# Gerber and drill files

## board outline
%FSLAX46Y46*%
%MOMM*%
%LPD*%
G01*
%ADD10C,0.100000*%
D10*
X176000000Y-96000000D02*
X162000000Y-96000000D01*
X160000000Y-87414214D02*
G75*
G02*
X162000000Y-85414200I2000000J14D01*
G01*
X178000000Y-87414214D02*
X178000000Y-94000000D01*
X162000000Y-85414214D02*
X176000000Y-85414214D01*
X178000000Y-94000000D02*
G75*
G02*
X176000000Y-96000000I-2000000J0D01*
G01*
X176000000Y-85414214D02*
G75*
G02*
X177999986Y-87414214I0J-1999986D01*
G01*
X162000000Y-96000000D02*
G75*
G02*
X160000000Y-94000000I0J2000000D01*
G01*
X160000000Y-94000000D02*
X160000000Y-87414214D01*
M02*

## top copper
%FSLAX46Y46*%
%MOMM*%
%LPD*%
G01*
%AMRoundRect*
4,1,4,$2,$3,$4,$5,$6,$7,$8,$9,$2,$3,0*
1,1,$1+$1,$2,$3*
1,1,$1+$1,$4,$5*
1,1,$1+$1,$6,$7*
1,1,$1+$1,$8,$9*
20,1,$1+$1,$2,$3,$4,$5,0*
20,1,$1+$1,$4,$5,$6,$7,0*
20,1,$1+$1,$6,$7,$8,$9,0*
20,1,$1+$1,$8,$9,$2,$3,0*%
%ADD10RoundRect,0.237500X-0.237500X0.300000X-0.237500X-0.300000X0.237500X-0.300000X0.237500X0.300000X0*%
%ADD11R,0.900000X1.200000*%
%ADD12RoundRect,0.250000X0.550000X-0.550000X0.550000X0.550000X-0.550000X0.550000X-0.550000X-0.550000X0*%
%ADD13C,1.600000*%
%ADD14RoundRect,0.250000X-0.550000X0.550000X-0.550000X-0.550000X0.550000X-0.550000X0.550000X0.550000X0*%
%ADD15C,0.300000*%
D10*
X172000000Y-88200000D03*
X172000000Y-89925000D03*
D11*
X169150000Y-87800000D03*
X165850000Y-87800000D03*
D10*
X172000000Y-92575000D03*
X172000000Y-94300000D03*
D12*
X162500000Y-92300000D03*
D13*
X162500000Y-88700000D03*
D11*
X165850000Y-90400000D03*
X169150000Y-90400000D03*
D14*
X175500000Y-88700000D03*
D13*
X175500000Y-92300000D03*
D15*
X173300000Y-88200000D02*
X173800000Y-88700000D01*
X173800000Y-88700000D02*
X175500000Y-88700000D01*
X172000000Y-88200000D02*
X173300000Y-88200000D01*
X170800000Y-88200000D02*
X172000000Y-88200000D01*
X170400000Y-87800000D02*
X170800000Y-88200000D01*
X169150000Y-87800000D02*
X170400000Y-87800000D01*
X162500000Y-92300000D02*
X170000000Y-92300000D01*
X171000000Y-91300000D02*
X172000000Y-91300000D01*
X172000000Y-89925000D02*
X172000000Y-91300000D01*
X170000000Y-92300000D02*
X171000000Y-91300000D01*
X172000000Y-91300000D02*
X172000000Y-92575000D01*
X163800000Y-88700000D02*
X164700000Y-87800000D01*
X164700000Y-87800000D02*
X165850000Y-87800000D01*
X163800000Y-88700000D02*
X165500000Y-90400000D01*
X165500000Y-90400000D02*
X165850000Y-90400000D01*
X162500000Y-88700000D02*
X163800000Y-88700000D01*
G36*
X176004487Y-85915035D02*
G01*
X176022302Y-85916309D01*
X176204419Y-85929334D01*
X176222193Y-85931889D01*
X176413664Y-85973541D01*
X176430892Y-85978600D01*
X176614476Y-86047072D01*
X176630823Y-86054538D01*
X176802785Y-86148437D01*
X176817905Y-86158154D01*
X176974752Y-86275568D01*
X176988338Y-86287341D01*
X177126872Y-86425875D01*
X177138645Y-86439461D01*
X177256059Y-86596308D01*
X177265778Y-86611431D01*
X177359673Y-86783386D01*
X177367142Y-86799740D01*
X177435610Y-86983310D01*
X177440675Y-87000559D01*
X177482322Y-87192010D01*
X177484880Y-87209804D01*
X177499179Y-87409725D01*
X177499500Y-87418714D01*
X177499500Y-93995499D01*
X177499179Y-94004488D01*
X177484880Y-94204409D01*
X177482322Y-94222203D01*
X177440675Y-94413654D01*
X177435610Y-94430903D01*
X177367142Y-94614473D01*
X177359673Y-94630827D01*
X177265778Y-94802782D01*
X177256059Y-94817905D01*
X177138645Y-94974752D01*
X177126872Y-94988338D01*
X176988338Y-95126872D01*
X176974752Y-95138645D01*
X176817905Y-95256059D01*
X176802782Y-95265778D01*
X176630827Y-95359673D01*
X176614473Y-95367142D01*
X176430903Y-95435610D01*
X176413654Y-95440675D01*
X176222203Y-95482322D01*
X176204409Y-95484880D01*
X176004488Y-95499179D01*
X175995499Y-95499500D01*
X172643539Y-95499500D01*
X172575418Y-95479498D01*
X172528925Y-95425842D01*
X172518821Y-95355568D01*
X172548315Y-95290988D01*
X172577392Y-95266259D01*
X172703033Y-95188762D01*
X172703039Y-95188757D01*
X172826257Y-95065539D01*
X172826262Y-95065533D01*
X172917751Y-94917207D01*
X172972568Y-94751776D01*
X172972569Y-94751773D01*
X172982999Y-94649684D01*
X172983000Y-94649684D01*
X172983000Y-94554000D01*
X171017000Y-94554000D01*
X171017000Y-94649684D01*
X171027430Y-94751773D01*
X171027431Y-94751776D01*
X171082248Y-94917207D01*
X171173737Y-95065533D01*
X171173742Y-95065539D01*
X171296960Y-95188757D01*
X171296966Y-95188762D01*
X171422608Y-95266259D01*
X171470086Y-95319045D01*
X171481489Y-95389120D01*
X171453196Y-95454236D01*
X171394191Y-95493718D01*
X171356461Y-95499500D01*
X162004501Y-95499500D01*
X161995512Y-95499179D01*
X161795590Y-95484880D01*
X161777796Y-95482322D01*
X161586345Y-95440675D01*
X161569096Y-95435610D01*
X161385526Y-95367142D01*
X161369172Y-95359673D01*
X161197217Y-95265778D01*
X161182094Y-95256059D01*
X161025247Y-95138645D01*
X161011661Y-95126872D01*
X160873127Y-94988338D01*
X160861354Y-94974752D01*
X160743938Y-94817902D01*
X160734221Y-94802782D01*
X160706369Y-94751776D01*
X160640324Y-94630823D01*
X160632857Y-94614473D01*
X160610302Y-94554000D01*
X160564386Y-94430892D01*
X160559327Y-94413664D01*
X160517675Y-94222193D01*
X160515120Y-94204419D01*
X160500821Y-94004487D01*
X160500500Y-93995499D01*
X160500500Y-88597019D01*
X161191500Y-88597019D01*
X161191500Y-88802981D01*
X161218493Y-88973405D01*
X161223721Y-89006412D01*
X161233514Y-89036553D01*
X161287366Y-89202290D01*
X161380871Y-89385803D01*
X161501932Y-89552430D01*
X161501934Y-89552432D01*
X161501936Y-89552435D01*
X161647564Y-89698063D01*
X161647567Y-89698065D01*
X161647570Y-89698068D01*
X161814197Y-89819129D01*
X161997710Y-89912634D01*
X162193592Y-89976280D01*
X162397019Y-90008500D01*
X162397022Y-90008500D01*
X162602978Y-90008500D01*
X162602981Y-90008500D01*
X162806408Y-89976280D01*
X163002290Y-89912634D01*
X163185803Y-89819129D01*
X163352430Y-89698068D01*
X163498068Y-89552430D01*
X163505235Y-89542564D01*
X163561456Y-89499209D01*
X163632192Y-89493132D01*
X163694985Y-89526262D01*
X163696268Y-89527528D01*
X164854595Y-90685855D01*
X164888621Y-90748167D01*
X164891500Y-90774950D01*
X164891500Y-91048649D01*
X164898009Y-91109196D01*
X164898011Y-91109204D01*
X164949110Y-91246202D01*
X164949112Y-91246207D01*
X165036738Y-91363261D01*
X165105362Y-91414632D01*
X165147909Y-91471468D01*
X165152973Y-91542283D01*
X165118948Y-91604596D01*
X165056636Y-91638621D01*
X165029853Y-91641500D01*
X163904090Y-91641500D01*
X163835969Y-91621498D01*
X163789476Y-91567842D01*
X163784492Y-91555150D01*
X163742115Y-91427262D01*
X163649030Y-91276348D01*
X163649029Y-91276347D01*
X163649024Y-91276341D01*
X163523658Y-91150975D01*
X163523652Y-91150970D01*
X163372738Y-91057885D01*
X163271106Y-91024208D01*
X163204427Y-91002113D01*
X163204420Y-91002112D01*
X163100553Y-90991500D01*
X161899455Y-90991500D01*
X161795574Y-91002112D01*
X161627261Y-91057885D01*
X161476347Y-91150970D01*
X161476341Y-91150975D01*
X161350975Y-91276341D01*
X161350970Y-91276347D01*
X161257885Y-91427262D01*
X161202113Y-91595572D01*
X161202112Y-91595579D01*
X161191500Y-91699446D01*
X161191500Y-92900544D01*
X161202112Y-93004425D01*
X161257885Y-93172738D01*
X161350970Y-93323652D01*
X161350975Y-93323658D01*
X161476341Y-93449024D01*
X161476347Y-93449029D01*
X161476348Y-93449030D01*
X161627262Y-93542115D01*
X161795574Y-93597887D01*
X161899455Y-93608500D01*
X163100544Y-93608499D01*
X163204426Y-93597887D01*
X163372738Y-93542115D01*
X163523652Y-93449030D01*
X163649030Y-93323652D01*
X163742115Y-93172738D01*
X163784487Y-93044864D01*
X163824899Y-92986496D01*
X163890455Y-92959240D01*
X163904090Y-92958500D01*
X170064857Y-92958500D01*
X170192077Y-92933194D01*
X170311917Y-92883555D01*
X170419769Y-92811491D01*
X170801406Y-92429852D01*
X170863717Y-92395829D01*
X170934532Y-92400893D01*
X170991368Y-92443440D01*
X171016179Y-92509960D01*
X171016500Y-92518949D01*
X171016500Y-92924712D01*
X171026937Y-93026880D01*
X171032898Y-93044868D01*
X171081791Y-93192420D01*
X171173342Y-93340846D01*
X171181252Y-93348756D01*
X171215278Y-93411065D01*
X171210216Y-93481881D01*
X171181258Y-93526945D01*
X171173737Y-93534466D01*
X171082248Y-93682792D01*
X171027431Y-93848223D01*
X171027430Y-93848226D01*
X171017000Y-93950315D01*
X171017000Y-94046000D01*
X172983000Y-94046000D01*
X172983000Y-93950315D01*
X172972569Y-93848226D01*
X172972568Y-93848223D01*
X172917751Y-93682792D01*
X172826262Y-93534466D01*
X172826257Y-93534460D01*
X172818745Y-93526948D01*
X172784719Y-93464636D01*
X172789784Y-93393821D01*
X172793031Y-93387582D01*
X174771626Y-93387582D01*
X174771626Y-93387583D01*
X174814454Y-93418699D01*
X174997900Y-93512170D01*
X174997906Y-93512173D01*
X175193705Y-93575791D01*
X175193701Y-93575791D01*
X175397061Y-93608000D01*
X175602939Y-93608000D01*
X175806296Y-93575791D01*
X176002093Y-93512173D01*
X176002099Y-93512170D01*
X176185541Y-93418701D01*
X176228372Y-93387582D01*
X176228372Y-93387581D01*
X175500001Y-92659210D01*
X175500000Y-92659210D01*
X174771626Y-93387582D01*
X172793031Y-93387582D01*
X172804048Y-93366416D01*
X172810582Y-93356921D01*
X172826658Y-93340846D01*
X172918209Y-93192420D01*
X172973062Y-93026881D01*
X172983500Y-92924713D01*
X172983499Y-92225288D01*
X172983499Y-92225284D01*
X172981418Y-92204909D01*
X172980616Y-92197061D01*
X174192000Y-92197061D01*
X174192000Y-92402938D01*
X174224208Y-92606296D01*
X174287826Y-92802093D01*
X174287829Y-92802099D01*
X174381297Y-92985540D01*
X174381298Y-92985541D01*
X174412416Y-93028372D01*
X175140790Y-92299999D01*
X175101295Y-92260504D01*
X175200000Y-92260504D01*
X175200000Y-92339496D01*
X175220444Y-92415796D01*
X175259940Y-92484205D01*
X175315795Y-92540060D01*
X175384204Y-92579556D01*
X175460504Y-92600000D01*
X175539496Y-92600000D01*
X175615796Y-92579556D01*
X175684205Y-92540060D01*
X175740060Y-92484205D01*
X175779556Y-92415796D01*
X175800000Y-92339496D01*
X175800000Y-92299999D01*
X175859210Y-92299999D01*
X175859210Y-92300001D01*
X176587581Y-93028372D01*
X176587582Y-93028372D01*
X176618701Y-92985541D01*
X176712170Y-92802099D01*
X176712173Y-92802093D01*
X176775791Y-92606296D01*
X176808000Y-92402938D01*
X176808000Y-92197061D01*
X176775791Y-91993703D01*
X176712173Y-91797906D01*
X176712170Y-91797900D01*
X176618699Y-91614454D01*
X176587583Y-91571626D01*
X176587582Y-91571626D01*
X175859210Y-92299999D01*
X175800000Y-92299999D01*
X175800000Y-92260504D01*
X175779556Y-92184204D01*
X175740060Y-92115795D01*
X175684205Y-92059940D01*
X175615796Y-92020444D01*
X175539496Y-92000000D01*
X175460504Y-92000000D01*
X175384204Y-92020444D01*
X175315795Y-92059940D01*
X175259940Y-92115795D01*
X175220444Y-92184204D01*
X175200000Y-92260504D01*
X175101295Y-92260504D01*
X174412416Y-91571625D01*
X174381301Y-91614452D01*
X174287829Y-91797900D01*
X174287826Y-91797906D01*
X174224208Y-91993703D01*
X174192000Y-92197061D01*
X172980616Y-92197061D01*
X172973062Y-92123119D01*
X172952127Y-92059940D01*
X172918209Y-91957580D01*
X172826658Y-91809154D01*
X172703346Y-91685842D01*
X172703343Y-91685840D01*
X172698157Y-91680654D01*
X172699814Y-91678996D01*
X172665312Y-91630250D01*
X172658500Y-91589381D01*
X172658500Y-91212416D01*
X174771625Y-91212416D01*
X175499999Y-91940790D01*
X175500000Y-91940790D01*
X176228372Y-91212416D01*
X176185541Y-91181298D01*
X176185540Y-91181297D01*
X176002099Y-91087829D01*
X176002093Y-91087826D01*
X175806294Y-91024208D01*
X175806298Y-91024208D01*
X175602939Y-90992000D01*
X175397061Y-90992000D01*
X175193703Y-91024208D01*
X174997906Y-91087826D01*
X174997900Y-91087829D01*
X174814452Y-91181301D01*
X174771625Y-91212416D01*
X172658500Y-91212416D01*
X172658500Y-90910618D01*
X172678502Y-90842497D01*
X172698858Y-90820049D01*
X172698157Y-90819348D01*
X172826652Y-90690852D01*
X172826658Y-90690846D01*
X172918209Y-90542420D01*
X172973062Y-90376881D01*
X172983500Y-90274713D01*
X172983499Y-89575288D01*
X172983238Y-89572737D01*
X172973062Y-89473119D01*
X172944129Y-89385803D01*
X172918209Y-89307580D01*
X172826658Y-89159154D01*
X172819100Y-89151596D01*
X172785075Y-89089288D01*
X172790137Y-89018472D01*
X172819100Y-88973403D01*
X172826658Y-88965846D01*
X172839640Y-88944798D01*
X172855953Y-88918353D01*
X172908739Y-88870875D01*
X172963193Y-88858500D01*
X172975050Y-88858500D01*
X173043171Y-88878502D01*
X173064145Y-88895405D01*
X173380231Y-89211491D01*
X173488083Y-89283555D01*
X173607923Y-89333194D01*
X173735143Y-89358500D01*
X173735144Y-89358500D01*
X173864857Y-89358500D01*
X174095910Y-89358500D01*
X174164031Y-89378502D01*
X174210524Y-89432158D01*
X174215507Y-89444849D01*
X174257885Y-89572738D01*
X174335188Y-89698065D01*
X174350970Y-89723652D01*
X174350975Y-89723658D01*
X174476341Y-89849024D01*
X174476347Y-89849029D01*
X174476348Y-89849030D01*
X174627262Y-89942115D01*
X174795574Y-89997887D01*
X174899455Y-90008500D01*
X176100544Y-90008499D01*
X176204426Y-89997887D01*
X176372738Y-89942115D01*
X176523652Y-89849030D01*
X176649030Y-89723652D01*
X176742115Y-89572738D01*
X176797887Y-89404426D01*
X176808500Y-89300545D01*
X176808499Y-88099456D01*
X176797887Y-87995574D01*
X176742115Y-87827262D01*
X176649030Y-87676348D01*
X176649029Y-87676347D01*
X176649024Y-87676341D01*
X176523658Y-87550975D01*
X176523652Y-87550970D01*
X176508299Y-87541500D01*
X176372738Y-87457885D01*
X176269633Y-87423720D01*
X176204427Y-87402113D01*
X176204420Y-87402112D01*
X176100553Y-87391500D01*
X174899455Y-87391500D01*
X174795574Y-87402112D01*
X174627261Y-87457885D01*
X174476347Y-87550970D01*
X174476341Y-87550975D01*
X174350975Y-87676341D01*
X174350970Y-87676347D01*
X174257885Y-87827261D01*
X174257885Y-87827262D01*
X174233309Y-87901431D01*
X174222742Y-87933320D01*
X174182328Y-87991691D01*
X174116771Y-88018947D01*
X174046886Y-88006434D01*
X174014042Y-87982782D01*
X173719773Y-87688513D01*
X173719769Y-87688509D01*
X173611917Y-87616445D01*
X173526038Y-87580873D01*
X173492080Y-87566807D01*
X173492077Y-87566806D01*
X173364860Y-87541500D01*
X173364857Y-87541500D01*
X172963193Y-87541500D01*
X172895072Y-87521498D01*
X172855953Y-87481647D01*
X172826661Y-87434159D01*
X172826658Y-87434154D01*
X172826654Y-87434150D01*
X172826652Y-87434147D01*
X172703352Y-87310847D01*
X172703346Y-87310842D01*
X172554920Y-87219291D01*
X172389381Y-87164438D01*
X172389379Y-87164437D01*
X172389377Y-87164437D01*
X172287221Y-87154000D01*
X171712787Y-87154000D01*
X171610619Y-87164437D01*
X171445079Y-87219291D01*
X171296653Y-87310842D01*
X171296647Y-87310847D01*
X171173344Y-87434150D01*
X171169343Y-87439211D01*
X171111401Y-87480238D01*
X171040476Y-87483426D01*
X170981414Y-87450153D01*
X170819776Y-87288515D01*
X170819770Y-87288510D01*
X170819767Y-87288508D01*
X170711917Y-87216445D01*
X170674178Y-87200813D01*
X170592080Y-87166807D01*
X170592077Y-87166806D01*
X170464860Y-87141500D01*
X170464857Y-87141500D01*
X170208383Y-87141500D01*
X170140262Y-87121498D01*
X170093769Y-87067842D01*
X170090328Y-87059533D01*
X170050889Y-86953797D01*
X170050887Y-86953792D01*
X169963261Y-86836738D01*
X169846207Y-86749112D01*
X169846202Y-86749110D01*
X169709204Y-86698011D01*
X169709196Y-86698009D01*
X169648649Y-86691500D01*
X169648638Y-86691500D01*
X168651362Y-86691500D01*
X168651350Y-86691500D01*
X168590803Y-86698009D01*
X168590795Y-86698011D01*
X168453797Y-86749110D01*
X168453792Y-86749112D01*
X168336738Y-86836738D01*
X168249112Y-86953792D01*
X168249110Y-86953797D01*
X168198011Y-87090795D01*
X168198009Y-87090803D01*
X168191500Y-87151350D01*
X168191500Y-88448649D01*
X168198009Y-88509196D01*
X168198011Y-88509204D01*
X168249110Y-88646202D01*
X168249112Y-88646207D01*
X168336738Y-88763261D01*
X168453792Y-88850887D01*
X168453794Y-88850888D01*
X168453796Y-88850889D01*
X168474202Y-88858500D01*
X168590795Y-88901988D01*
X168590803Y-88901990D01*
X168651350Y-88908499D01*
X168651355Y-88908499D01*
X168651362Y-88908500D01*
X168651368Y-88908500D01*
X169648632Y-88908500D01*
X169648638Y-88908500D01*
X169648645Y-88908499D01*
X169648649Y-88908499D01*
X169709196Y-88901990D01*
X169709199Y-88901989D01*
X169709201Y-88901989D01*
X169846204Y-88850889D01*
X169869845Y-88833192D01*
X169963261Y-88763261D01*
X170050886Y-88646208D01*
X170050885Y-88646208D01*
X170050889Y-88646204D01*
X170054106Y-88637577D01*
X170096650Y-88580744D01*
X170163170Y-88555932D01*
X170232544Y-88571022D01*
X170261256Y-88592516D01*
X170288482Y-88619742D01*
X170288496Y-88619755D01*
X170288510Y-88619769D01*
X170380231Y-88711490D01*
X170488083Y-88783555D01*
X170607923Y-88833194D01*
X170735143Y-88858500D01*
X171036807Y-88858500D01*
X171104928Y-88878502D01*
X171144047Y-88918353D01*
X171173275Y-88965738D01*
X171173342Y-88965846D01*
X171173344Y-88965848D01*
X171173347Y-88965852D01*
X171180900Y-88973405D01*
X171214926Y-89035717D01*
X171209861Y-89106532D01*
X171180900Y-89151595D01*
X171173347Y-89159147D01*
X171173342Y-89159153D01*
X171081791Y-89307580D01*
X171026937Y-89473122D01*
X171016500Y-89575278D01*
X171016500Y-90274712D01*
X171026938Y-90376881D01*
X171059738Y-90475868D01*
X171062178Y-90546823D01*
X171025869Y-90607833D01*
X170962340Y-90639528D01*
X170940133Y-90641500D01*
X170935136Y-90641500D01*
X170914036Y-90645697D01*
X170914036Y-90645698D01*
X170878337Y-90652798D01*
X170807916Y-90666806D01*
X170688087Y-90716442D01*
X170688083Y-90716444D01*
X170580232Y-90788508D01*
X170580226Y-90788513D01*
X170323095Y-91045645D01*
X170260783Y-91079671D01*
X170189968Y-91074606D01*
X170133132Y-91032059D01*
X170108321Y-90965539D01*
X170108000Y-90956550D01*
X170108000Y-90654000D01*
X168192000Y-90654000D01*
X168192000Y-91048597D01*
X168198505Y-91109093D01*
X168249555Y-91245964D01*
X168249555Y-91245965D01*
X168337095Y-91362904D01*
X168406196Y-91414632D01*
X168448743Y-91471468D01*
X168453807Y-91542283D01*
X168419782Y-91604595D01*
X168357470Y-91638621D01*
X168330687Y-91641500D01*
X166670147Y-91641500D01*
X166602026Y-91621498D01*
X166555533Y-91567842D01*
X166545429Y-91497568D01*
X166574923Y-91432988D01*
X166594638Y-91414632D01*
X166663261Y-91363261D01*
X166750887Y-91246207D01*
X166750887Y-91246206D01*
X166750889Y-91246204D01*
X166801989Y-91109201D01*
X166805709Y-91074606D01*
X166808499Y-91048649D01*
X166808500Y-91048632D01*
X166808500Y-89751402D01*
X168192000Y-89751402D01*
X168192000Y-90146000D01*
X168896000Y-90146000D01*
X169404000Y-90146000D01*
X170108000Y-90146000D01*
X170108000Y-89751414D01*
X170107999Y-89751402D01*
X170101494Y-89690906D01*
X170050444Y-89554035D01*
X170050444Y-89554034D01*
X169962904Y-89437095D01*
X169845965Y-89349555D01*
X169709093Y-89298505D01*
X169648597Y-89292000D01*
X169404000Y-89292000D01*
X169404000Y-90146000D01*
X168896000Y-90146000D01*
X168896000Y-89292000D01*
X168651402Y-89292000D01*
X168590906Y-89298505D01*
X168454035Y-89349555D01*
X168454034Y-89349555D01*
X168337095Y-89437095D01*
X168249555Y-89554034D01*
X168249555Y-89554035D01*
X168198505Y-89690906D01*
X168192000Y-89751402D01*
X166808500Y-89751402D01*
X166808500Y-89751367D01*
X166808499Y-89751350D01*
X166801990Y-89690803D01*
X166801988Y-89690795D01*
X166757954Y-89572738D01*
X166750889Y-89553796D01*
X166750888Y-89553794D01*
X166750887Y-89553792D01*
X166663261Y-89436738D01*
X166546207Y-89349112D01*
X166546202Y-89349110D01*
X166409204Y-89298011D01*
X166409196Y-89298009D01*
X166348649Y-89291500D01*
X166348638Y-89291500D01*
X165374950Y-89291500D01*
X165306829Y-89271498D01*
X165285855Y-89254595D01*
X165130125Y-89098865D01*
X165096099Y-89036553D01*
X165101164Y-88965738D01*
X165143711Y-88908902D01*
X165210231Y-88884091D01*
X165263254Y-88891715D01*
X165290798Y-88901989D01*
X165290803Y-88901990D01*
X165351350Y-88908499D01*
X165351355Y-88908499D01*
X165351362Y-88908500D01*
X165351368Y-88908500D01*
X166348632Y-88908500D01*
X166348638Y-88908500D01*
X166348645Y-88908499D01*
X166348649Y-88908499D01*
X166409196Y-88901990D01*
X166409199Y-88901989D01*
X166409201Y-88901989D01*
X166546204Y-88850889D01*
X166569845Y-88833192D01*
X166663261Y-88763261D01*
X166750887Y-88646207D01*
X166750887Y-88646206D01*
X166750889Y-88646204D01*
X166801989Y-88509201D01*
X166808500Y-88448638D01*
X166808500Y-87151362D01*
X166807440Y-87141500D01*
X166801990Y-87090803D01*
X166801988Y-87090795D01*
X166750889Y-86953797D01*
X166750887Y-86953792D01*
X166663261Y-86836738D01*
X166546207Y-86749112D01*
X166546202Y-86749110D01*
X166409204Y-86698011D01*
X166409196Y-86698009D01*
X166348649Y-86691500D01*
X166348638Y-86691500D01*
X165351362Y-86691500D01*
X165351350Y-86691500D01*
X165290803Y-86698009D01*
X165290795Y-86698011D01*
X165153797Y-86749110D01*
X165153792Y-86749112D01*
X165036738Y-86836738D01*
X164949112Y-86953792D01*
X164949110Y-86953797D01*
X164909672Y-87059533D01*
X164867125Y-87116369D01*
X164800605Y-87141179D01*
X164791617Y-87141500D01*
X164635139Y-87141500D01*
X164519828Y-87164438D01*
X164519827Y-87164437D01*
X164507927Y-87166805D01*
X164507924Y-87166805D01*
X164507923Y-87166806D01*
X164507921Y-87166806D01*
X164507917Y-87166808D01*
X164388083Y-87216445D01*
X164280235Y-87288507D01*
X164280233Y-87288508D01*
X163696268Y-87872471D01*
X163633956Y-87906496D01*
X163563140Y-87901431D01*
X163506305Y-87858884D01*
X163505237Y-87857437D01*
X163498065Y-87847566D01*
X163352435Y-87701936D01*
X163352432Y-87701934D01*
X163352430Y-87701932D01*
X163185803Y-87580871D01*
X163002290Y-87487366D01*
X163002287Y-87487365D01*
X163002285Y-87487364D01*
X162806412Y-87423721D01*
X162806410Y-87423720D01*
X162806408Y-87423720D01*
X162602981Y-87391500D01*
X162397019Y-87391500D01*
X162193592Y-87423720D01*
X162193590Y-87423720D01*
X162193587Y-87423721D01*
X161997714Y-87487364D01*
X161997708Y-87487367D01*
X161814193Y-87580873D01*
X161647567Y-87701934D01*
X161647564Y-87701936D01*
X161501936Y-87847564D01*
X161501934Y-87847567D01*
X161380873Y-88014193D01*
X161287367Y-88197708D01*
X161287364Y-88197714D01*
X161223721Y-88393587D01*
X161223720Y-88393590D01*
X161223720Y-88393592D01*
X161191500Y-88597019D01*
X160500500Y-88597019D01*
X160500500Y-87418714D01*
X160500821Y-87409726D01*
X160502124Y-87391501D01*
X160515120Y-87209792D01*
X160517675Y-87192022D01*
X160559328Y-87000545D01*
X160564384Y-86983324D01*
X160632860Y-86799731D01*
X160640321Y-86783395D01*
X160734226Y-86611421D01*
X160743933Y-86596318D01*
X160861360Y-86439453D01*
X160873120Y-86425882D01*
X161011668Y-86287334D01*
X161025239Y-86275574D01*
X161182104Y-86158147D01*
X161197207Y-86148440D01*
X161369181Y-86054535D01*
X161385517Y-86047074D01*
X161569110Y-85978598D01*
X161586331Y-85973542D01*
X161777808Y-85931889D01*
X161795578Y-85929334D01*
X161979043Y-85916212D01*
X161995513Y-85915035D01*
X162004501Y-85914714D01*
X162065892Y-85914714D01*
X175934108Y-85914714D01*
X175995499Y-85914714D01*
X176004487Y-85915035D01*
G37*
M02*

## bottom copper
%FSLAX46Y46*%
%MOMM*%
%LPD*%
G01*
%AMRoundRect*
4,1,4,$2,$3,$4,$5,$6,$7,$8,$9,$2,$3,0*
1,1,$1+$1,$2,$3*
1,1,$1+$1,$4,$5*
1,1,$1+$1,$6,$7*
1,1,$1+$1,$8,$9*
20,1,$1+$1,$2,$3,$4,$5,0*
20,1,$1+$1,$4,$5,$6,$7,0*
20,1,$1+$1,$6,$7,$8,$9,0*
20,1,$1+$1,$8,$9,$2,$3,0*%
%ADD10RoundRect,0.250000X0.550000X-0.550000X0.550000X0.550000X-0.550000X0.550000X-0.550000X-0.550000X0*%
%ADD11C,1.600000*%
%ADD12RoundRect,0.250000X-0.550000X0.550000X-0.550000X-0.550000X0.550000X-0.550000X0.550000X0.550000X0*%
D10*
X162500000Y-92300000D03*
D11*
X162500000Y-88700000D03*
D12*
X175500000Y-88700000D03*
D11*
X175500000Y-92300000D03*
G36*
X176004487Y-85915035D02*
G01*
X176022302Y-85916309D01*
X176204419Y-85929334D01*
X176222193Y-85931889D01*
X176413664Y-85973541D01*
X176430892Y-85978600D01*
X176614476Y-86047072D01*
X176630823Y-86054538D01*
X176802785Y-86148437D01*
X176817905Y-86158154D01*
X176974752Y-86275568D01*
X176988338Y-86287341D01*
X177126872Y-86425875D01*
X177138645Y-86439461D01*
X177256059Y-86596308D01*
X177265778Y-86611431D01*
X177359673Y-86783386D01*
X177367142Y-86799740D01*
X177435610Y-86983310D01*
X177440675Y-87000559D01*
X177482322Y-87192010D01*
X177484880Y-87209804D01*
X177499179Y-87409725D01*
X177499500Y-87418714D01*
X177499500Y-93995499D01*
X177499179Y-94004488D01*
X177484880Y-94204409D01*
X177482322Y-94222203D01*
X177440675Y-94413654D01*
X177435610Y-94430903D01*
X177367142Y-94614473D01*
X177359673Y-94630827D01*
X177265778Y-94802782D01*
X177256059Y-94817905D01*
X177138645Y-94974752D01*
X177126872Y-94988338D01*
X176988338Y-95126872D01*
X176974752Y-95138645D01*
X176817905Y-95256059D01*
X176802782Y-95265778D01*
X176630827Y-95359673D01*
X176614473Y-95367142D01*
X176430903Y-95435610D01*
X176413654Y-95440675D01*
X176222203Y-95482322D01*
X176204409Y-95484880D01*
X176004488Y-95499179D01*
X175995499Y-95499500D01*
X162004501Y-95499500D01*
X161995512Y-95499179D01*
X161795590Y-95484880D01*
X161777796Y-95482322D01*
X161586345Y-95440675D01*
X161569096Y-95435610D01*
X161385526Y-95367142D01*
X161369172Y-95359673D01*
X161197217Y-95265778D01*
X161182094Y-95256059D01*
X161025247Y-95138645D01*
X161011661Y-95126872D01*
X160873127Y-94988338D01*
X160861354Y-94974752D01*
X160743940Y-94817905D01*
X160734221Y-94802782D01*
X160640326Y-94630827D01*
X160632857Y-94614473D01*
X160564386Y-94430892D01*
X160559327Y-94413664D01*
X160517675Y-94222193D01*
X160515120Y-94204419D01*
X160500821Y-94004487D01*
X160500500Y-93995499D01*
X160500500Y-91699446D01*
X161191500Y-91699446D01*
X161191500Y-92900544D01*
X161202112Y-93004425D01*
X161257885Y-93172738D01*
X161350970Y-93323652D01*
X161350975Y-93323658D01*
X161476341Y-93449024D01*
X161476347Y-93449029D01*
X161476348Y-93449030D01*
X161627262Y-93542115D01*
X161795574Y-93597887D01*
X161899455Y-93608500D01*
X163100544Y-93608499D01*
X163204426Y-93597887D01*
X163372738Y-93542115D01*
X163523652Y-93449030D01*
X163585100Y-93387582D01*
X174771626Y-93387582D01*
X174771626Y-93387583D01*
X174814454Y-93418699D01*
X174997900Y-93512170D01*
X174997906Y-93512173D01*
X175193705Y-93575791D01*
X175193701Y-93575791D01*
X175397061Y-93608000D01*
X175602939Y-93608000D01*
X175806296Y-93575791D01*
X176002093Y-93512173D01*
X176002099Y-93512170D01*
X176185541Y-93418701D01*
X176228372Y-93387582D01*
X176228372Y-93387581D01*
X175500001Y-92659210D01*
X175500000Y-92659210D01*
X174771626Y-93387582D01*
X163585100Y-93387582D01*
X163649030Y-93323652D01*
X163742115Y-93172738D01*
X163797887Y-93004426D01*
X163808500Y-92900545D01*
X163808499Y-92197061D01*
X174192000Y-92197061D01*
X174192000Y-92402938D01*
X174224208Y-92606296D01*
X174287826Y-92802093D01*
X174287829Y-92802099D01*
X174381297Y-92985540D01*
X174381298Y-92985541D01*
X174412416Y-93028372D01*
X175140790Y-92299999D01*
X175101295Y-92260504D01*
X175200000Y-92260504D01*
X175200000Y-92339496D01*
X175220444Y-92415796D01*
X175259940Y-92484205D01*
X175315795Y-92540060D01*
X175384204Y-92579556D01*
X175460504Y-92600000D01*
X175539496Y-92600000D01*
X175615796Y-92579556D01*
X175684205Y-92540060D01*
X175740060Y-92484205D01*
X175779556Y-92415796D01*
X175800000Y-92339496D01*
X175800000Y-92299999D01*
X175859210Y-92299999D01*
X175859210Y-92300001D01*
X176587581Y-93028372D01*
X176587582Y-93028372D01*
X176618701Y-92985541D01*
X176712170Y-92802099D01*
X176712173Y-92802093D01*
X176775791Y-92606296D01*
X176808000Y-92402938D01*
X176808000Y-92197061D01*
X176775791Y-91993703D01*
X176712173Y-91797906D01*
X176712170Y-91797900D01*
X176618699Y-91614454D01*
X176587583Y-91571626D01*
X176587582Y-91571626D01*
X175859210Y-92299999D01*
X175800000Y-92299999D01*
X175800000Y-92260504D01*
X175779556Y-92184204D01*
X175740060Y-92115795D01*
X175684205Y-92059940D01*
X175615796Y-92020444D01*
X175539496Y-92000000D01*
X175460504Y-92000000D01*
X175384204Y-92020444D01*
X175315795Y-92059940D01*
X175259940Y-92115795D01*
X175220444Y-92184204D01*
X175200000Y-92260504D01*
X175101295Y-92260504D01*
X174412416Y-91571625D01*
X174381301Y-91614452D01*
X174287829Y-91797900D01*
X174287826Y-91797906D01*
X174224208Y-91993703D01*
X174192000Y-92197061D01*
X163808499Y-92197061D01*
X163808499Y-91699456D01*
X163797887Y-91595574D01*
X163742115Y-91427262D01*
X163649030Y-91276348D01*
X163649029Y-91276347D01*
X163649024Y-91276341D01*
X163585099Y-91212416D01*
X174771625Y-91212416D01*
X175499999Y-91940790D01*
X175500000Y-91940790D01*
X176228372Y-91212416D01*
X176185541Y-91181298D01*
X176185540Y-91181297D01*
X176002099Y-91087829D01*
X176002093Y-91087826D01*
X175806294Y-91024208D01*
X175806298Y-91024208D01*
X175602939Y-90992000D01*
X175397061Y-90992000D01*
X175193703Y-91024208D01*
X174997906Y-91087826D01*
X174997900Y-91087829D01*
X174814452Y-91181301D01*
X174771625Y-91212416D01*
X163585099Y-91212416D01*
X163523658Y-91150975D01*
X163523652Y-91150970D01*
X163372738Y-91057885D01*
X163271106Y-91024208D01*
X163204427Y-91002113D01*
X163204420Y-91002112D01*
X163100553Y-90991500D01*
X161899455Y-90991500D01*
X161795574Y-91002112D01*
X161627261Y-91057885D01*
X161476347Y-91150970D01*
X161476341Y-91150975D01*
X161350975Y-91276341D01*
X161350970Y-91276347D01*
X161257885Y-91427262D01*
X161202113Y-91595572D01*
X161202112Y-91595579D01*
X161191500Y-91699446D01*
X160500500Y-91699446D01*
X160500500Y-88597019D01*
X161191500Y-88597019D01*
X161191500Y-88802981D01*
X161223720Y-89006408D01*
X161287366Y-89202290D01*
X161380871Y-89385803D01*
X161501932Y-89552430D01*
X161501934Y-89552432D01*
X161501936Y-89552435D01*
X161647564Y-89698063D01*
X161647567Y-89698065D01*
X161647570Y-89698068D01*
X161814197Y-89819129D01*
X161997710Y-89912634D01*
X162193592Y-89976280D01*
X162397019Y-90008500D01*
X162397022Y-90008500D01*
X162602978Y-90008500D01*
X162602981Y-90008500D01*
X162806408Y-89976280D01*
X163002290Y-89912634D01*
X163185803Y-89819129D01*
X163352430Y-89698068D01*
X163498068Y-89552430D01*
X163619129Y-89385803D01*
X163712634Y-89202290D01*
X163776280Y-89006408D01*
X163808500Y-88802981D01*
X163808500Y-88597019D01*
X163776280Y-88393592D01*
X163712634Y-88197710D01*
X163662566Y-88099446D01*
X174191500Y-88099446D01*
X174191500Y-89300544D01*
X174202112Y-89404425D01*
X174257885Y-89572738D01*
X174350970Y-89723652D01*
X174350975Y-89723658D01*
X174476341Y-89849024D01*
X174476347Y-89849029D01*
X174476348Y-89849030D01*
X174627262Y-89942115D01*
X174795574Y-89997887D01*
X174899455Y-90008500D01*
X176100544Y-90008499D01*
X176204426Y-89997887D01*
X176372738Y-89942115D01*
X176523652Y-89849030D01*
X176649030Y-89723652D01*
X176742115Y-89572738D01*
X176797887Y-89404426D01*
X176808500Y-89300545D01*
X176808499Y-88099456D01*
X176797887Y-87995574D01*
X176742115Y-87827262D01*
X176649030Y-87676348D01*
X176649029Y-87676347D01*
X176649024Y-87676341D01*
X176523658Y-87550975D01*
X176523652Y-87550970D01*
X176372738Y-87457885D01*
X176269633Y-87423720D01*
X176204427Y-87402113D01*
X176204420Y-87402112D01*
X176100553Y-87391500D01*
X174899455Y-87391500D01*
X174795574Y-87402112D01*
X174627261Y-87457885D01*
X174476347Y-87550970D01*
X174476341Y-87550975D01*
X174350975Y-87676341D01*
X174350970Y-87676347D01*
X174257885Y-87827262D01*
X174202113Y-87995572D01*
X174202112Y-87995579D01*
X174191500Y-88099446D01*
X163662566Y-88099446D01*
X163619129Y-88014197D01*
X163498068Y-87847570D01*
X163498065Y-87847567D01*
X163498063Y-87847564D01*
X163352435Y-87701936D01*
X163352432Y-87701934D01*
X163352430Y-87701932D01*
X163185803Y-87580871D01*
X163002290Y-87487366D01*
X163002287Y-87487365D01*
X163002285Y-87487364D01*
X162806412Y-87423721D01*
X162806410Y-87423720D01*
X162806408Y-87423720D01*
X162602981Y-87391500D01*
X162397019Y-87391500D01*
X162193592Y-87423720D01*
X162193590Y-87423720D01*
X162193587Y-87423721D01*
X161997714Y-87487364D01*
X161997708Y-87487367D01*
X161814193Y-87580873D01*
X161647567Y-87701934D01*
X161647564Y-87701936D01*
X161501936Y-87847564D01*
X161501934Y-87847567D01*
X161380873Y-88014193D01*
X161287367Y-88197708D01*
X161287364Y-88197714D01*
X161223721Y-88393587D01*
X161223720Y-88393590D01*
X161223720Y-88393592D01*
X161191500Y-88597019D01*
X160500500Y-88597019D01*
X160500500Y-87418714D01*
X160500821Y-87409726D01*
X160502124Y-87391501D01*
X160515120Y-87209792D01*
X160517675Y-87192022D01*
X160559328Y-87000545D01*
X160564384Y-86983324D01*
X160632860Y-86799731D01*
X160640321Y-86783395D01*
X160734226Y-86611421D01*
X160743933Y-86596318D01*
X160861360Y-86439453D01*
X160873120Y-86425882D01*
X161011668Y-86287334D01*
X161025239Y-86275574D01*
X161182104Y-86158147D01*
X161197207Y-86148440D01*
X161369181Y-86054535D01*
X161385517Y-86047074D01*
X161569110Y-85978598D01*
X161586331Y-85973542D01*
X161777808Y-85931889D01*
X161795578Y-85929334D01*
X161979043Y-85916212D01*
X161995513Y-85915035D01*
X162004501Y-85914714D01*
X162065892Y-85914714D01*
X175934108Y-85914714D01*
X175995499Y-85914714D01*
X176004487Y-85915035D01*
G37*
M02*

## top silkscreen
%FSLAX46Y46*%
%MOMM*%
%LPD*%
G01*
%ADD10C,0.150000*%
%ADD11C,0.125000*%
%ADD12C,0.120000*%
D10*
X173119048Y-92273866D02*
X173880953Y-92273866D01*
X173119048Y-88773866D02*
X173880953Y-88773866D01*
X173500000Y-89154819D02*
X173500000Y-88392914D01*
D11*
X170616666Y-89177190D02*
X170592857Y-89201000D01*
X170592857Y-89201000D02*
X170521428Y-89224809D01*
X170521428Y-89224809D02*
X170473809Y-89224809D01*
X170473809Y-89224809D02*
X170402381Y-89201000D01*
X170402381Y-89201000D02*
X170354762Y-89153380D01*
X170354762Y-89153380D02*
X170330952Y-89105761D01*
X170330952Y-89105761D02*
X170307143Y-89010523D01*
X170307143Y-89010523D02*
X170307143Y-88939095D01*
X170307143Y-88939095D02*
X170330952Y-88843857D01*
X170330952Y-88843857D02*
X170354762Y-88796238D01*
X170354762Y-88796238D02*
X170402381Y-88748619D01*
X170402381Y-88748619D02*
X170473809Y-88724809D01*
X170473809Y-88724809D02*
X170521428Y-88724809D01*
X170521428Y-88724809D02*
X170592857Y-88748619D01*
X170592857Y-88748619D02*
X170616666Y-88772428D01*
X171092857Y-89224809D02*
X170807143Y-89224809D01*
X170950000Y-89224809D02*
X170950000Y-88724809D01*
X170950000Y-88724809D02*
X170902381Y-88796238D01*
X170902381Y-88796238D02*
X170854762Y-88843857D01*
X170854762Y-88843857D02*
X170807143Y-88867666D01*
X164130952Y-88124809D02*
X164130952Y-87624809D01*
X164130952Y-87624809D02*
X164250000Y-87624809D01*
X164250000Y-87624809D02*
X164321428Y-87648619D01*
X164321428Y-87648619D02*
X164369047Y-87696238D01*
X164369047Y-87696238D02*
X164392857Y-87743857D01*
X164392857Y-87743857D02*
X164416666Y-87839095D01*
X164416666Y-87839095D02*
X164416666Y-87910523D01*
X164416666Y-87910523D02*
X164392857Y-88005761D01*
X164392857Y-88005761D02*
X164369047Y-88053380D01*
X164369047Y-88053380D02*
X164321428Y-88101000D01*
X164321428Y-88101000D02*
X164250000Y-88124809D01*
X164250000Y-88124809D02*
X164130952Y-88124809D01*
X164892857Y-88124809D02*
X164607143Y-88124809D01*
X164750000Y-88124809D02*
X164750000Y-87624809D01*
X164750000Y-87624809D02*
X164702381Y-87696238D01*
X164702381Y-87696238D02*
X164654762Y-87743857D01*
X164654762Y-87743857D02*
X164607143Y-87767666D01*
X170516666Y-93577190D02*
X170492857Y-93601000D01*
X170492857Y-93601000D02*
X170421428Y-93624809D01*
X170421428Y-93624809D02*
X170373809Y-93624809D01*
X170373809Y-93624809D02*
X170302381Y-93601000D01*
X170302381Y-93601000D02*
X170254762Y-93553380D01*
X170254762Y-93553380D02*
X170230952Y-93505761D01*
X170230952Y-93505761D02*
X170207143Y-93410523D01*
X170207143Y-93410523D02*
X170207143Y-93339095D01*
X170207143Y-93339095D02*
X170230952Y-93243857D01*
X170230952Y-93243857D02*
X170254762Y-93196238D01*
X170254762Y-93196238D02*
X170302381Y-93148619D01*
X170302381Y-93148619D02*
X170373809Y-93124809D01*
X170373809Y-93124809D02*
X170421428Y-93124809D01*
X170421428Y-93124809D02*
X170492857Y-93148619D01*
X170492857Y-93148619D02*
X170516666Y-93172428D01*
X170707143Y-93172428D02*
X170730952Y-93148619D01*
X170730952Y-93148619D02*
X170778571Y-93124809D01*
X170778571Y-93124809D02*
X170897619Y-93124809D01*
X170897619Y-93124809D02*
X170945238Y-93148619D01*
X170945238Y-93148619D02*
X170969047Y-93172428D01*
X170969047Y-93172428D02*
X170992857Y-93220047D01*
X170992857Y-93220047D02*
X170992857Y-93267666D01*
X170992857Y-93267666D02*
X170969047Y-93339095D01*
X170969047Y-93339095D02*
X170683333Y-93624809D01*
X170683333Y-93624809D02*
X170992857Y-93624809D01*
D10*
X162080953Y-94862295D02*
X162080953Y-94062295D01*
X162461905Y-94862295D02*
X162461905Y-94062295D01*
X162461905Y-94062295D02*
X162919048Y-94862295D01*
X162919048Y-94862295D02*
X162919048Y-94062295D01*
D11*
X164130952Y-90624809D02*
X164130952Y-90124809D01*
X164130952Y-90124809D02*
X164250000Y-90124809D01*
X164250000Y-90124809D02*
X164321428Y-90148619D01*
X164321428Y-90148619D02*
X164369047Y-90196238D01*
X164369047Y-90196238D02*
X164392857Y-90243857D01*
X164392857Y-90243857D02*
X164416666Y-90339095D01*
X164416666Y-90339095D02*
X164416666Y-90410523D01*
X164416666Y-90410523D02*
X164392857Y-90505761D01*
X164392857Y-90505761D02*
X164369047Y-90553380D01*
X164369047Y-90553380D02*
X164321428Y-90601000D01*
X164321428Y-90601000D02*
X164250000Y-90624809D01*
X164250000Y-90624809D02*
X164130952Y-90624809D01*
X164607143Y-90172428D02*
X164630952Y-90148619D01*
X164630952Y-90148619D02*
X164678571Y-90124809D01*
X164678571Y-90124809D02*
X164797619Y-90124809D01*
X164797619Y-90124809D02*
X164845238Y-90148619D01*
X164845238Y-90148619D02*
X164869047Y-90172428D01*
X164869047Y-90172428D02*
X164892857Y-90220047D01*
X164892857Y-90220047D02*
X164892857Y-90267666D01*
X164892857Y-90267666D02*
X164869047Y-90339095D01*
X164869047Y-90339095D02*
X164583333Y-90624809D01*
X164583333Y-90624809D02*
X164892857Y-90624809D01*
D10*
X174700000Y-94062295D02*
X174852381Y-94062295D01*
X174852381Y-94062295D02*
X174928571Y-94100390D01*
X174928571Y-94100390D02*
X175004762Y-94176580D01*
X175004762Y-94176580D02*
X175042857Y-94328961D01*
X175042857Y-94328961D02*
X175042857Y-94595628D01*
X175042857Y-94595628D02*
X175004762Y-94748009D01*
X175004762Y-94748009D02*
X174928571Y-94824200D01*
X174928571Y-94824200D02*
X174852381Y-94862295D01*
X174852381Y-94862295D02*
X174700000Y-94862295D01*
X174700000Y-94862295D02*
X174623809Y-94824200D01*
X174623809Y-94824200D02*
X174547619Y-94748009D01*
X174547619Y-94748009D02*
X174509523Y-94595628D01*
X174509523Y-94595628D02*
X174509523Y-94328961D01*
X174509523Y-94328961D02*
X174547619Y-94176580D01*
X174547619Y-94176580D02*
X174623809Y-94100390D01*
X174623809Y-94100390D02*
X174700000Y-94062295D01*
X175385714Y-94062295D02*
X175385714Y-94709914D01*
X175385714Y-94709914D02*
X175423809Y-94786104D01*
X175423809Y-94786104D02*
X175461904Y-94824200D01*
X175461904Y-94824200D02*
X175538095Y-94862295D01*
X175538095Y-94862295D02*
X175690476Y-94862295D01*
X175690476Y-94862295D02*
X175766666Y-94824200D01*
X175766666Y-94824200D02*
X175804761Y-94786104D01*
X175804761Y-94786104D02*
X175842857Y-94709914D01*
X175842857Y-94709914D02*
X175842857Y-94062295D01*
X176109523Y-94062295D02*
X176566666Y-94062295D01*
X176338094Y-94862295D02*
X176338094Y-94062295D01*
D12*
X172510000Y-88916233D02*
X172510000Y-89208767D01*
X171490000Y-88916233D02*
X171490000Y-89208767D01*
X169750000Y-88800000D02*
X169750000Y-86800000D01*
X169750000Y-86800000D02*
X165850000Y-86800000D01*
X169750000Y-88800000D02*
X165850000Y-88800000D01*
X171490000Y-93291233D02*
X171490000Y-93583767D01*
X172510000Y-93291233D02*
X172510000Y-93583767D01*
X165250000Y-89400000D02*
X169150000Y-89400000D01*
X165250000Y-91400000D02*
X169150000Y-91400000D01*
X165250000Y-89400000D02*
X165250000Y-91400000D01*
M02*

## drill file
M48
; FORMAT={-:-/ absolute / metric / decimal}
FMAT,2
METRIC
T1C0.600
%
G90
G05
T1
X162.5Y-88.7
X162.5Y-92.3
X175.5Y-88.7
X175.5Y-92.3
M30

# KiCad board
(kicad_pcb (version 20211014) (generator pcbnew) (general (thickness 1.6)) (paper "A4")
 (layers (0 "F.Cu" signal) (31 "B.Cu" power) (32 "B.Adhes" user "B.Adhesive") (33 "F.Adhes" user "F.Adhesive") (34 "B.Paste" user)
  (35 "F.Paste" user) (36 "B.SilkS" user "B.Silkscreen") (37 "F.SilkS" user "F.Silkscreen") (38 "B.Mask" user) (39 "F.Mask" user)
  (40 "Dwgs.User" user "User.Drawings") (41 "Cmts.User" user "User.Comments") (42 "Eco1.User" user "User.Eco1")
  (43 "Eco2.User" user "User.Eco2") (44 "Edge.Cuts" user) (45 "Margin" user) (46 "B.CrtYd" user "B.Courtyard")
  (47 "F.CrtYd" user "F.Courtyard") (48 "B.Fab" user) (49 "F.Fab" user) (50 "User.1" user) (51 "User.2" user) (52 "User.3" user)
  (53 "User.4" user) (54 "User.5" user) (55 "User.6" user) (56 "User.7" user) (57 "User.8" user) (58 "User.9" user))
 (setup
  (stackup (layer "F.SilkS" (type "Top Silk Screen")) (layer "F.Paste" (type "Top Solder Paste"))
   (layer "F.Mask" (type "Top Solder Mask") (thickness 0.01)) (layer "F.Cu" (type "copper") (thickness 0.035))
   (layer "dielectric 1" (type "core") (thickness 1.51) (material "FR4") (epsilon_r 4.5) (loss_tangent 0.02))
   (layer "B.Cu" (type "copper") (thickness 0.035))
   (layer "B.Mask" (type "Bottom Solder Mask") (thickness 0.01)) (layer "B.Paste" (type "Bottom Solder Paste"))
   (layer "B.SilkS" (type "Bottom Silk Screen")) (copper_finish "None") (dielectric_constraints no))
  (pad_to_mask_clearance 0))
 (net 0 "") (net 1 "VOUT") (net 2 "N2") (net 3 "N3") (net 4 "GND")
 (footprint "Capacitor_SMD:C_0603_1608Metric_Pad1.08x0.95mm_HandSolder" (layer "F.Cu") (at 172 89.0625 -90)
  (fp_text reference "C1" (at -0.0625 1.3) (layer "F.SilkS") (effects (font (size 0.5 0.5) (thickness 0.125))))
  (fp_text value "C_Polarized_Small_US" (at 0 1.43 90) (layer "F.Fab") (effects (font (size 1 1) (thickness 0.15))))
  (fp_line (start -0.146267 -0.51) (end 0.146267 -0.51) (layer "F.SilkS") (width 0.12))
  (fp_line (start -0.146267 0.51) (end 0.146267 0.51) (layer "F.SilkS") (width 0.12))
  (pad "1" smd roundrect (at -0.8625 0 270) (size 1.075 0.95) (layers "F.Cu" "F.Paste" "F.Mask") (roundrect_rratio 0.25) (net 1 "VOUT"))
  (pad "2" smd roundrect (at 0.8625 0 270) (size 1.075 0.95) (layers "F.Cu" "F.Paste" "F.Mask") (roundrect_rratio 0.25) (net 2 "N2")))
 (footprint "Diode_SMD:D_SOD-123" (layer "F.Cu") (at 167.5 87.8 180)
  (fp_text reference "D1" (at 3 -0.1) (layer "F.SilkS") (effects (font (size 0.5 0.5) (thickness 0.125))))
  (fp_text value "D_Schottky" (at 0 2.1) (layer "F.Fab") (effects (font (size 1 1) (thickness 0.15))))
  (fp_line (start -2.25 -1) (end -2.25 1) (layer "F.SilkS") (width 0.12))
  (fp_line (start -2.25 1) (end 1.65 1) (layer "F.SilkS") (width 0.12))
  (fp_line (start -2.25 -1) (end 1.65 -1) (layer "F.SilkS") (width 0.12))
  (pad "1" smd rect (at -1.65 0 180) (size 0.9 1.2) (layers "F.Cu" "F.Paste" "F.Mask") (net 1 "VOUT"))
  (pad "2" smd rect (at 1.65 0 180) (size 0.9 1.2) (layers "F.Cu" "F.Paste" "F.Mask") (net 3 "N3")))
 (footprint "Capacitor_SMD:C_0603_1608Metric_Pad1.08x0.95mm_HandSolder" (layer "F.Cu") (at 172 93.4375 -90)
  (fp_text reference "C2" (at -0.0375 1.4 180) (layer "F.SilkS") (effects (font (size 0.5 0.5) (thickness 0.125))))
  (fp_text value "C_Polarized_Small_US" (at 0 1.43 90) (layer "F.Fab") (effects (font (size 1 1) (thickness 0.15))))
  (fp_line (start -0.146267 0.51) (end 0.146267 0.51) (layer "F.SilkS") (width 0.12))
  (fp_line (start -0.146267 -0.51) (end 0.146267 -0.51) (layer "F.SilkS") (width 0.12))
  (pad "1" smd roundrect (at -0.8625 0 270) (size 1.075 0.95) (layers "F.Cu" "F.Paste" "F.Mask") (roundrect_rratio 0.25) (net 2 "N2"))
  (pad "2" smd roundrect (at 0.8625 0 270) (size 1.075 0.95) (layers "F.Cu" "F.Paste" "F.Mask") (roundrect_rratio 0.25) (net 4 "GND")))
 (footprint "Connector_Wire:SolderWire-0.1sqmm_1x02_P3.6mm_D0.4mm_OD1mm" (layer "F.Cu") (at 162.5 92.3 90)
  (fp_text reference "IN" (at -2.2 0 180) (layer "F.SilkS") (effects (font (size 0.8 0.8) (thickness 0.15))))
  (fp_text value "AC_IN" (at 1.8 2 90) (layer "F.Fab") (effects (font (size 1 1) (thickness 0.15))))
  (pad "1" thru_hole roundrect (at 0 0 90) (size 1.6 1.6) (drill 0.6) (layers *.Cu *.Mask) (roundrect_rratio 0.15625) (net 2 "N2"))
  (pad "2" thru_hole circle (at 3.6 0 90) (size 1.6 1.6) (drill 0.6) (layers *.Cu *.Mask) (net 3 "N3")))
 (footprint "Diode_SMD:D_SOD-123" (layer "F.Cu") (at 167.5 90.4)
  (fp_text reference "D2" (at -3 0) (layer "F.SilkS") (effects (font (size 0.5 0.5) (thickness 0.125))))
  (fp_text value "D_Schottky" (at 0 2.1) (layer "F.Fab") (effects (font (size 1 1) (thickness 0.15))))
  (fp_line (start -2.25 -1) (end 1.65 -1) (layer "F.SilkS") (width 0.12))
  (fp_line (start -2.25 1) (end 1.65 1) (layer "F.SilkS") (width 0.12))
  (fp_line (start -2.25 -1) (end -2.25 1) (layer "F.SilkS") (width 0.12))
  (pad "1" smd rect (at -1.65 0) (size 0.9 1.2) (layers "F.Cu" "F.Paste" "F.Mask") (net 3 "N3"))
  (pad "2" smd rect (at 1.65 0) (size 0.9 1.2) (layers "F.Cu" "F.Paste" "F.Mask") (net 4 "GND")))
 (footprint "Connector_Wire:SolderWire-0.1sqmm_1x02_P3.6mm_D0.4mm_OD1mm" (layer "F.Cu") (at 175.5 88.7 -90)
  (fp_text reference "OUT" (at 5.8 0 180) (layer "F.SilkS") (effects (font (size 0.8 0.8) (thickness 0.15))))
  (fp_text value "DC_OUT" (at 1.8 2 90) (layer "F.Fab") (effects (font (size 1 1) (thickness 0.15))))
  (pad "1" thru_hole roundrect (at 0 0 270) (size 1.6 1.6) (drill 0.6) (layers *.Cu *.Mask) (roundrect_rratio 0.15625) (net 1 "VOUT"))
  (pad "2" thru_hole circle (at 3.6 0 270) (size 1.6 1.6) (drill 0.6) (layers *.Cu *.Mask) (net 4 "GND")))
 (gr_line (start 176 96) (end 162 96) (layer "Edge.Cuts") (width 0.1))
 (gr_arc (start 160 87.414214) (mid 160.585786 86) (end 162 85.414214) (layer "Edge.Cuts") (width 0.1))
 (gr_line (start 178 87.414214) (end 178 94) (layer "Edge.Cuts") (width 0.1))
 (gr_line (start 162 85.414214) (end 176 85.414214) (layer "Edge.Cuts") (width 0.1))
 (gr_arc (start 178 94) (mid 177.414214 95.414214) (end 176 96) (layer "Edge.Cuts") (width 0.1))
 (gr_arc (start 176 85.414214) (mid 177.414214 86) (end 178 87.414214) (layer "Edge.Cuts") (width 0.1))
 (gr_arc (start 162 96) (mid 160.585786 95.414214) (end 160 94) (layer "Edge.Cuts") (width 0.1))
 (gr_line (start 160 94) (end 160 87.414214) (layer "Edge.Cuts") (width 0.1))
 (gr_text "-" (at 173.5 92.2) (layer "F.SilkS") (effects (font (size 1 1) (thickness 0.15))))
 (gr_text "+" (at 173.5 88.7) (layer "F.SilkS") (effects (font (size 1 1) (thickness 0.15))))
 (segment (start 173.3 88.2) (end 173.8 88.7) (width 0.3) (layer "F.Cu") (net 1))
 (segment (start 173.8 88.7) (end 175.5 88.7) (width 0.3) (layer "F.Cu") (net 1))
 (segment (start 172 88.2) (end 173.3 88.2) (width 0.3) (layer "F.Cu") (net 1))
 (segment (start 170.8 88.2) (end 172 88.2) (width 0.3) (layer "F.Cu") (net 1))
 (segment (start 170.4 87.8) (end 170.8 88.2) (width 0.3) (layer "F.Cu") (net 1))
 (segment (start 169.15 87.8) (end 170.4 87.8) (width 0.3) (layer "F.Cu") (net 1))
 (segment (start 162.5 92.3) (end 170 92.3) (width 0.3) (layer "F.Cu") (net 2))
 (segment (start 171 91.3) (end 172 91.3) (width 0.3) (layer "F.Cu") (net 2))
 (segment (start 172 89.925) (end 172 91.3) (width 0.3) (layer "F.Cu") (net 2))
 (segment (start 170 92.3) (end 171 91.3) (width 0.3) (layer "F.Cu") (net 2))
 (segment (start 172 91.3) (end 172 92.575) (width 0.3) (layer "F.Cu") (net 2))
 (segment (start 163.8 88.7) (end 164.7 87.8) (width 0.3) (layer "F.Cu") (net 3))
 (segment (start 164.7 87.8) (end 165.85 87.8) (width 0.3) (layer "F.Cu") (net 3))
 (segment (start 163.8 88.7) (end 165.5 90.4) (width 0.3) (layer "F.Cu") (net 3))
 (segment (start 165.5 90.4) (end 165.85 90.4) (width 0.3) (layer "F.Cu") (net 3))
 (segment (start 162.5 88.7) (end 163.8 88.7) (width 0.3) (layer "F.Cu") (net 3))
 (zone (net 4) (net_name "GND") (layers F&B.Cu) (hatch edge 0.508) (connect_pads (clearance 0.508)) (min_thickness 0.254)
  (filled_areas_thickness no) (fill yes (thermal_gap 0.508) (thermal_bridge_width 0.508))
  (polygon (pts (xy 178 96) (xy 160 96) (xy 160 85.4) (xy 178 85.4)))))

